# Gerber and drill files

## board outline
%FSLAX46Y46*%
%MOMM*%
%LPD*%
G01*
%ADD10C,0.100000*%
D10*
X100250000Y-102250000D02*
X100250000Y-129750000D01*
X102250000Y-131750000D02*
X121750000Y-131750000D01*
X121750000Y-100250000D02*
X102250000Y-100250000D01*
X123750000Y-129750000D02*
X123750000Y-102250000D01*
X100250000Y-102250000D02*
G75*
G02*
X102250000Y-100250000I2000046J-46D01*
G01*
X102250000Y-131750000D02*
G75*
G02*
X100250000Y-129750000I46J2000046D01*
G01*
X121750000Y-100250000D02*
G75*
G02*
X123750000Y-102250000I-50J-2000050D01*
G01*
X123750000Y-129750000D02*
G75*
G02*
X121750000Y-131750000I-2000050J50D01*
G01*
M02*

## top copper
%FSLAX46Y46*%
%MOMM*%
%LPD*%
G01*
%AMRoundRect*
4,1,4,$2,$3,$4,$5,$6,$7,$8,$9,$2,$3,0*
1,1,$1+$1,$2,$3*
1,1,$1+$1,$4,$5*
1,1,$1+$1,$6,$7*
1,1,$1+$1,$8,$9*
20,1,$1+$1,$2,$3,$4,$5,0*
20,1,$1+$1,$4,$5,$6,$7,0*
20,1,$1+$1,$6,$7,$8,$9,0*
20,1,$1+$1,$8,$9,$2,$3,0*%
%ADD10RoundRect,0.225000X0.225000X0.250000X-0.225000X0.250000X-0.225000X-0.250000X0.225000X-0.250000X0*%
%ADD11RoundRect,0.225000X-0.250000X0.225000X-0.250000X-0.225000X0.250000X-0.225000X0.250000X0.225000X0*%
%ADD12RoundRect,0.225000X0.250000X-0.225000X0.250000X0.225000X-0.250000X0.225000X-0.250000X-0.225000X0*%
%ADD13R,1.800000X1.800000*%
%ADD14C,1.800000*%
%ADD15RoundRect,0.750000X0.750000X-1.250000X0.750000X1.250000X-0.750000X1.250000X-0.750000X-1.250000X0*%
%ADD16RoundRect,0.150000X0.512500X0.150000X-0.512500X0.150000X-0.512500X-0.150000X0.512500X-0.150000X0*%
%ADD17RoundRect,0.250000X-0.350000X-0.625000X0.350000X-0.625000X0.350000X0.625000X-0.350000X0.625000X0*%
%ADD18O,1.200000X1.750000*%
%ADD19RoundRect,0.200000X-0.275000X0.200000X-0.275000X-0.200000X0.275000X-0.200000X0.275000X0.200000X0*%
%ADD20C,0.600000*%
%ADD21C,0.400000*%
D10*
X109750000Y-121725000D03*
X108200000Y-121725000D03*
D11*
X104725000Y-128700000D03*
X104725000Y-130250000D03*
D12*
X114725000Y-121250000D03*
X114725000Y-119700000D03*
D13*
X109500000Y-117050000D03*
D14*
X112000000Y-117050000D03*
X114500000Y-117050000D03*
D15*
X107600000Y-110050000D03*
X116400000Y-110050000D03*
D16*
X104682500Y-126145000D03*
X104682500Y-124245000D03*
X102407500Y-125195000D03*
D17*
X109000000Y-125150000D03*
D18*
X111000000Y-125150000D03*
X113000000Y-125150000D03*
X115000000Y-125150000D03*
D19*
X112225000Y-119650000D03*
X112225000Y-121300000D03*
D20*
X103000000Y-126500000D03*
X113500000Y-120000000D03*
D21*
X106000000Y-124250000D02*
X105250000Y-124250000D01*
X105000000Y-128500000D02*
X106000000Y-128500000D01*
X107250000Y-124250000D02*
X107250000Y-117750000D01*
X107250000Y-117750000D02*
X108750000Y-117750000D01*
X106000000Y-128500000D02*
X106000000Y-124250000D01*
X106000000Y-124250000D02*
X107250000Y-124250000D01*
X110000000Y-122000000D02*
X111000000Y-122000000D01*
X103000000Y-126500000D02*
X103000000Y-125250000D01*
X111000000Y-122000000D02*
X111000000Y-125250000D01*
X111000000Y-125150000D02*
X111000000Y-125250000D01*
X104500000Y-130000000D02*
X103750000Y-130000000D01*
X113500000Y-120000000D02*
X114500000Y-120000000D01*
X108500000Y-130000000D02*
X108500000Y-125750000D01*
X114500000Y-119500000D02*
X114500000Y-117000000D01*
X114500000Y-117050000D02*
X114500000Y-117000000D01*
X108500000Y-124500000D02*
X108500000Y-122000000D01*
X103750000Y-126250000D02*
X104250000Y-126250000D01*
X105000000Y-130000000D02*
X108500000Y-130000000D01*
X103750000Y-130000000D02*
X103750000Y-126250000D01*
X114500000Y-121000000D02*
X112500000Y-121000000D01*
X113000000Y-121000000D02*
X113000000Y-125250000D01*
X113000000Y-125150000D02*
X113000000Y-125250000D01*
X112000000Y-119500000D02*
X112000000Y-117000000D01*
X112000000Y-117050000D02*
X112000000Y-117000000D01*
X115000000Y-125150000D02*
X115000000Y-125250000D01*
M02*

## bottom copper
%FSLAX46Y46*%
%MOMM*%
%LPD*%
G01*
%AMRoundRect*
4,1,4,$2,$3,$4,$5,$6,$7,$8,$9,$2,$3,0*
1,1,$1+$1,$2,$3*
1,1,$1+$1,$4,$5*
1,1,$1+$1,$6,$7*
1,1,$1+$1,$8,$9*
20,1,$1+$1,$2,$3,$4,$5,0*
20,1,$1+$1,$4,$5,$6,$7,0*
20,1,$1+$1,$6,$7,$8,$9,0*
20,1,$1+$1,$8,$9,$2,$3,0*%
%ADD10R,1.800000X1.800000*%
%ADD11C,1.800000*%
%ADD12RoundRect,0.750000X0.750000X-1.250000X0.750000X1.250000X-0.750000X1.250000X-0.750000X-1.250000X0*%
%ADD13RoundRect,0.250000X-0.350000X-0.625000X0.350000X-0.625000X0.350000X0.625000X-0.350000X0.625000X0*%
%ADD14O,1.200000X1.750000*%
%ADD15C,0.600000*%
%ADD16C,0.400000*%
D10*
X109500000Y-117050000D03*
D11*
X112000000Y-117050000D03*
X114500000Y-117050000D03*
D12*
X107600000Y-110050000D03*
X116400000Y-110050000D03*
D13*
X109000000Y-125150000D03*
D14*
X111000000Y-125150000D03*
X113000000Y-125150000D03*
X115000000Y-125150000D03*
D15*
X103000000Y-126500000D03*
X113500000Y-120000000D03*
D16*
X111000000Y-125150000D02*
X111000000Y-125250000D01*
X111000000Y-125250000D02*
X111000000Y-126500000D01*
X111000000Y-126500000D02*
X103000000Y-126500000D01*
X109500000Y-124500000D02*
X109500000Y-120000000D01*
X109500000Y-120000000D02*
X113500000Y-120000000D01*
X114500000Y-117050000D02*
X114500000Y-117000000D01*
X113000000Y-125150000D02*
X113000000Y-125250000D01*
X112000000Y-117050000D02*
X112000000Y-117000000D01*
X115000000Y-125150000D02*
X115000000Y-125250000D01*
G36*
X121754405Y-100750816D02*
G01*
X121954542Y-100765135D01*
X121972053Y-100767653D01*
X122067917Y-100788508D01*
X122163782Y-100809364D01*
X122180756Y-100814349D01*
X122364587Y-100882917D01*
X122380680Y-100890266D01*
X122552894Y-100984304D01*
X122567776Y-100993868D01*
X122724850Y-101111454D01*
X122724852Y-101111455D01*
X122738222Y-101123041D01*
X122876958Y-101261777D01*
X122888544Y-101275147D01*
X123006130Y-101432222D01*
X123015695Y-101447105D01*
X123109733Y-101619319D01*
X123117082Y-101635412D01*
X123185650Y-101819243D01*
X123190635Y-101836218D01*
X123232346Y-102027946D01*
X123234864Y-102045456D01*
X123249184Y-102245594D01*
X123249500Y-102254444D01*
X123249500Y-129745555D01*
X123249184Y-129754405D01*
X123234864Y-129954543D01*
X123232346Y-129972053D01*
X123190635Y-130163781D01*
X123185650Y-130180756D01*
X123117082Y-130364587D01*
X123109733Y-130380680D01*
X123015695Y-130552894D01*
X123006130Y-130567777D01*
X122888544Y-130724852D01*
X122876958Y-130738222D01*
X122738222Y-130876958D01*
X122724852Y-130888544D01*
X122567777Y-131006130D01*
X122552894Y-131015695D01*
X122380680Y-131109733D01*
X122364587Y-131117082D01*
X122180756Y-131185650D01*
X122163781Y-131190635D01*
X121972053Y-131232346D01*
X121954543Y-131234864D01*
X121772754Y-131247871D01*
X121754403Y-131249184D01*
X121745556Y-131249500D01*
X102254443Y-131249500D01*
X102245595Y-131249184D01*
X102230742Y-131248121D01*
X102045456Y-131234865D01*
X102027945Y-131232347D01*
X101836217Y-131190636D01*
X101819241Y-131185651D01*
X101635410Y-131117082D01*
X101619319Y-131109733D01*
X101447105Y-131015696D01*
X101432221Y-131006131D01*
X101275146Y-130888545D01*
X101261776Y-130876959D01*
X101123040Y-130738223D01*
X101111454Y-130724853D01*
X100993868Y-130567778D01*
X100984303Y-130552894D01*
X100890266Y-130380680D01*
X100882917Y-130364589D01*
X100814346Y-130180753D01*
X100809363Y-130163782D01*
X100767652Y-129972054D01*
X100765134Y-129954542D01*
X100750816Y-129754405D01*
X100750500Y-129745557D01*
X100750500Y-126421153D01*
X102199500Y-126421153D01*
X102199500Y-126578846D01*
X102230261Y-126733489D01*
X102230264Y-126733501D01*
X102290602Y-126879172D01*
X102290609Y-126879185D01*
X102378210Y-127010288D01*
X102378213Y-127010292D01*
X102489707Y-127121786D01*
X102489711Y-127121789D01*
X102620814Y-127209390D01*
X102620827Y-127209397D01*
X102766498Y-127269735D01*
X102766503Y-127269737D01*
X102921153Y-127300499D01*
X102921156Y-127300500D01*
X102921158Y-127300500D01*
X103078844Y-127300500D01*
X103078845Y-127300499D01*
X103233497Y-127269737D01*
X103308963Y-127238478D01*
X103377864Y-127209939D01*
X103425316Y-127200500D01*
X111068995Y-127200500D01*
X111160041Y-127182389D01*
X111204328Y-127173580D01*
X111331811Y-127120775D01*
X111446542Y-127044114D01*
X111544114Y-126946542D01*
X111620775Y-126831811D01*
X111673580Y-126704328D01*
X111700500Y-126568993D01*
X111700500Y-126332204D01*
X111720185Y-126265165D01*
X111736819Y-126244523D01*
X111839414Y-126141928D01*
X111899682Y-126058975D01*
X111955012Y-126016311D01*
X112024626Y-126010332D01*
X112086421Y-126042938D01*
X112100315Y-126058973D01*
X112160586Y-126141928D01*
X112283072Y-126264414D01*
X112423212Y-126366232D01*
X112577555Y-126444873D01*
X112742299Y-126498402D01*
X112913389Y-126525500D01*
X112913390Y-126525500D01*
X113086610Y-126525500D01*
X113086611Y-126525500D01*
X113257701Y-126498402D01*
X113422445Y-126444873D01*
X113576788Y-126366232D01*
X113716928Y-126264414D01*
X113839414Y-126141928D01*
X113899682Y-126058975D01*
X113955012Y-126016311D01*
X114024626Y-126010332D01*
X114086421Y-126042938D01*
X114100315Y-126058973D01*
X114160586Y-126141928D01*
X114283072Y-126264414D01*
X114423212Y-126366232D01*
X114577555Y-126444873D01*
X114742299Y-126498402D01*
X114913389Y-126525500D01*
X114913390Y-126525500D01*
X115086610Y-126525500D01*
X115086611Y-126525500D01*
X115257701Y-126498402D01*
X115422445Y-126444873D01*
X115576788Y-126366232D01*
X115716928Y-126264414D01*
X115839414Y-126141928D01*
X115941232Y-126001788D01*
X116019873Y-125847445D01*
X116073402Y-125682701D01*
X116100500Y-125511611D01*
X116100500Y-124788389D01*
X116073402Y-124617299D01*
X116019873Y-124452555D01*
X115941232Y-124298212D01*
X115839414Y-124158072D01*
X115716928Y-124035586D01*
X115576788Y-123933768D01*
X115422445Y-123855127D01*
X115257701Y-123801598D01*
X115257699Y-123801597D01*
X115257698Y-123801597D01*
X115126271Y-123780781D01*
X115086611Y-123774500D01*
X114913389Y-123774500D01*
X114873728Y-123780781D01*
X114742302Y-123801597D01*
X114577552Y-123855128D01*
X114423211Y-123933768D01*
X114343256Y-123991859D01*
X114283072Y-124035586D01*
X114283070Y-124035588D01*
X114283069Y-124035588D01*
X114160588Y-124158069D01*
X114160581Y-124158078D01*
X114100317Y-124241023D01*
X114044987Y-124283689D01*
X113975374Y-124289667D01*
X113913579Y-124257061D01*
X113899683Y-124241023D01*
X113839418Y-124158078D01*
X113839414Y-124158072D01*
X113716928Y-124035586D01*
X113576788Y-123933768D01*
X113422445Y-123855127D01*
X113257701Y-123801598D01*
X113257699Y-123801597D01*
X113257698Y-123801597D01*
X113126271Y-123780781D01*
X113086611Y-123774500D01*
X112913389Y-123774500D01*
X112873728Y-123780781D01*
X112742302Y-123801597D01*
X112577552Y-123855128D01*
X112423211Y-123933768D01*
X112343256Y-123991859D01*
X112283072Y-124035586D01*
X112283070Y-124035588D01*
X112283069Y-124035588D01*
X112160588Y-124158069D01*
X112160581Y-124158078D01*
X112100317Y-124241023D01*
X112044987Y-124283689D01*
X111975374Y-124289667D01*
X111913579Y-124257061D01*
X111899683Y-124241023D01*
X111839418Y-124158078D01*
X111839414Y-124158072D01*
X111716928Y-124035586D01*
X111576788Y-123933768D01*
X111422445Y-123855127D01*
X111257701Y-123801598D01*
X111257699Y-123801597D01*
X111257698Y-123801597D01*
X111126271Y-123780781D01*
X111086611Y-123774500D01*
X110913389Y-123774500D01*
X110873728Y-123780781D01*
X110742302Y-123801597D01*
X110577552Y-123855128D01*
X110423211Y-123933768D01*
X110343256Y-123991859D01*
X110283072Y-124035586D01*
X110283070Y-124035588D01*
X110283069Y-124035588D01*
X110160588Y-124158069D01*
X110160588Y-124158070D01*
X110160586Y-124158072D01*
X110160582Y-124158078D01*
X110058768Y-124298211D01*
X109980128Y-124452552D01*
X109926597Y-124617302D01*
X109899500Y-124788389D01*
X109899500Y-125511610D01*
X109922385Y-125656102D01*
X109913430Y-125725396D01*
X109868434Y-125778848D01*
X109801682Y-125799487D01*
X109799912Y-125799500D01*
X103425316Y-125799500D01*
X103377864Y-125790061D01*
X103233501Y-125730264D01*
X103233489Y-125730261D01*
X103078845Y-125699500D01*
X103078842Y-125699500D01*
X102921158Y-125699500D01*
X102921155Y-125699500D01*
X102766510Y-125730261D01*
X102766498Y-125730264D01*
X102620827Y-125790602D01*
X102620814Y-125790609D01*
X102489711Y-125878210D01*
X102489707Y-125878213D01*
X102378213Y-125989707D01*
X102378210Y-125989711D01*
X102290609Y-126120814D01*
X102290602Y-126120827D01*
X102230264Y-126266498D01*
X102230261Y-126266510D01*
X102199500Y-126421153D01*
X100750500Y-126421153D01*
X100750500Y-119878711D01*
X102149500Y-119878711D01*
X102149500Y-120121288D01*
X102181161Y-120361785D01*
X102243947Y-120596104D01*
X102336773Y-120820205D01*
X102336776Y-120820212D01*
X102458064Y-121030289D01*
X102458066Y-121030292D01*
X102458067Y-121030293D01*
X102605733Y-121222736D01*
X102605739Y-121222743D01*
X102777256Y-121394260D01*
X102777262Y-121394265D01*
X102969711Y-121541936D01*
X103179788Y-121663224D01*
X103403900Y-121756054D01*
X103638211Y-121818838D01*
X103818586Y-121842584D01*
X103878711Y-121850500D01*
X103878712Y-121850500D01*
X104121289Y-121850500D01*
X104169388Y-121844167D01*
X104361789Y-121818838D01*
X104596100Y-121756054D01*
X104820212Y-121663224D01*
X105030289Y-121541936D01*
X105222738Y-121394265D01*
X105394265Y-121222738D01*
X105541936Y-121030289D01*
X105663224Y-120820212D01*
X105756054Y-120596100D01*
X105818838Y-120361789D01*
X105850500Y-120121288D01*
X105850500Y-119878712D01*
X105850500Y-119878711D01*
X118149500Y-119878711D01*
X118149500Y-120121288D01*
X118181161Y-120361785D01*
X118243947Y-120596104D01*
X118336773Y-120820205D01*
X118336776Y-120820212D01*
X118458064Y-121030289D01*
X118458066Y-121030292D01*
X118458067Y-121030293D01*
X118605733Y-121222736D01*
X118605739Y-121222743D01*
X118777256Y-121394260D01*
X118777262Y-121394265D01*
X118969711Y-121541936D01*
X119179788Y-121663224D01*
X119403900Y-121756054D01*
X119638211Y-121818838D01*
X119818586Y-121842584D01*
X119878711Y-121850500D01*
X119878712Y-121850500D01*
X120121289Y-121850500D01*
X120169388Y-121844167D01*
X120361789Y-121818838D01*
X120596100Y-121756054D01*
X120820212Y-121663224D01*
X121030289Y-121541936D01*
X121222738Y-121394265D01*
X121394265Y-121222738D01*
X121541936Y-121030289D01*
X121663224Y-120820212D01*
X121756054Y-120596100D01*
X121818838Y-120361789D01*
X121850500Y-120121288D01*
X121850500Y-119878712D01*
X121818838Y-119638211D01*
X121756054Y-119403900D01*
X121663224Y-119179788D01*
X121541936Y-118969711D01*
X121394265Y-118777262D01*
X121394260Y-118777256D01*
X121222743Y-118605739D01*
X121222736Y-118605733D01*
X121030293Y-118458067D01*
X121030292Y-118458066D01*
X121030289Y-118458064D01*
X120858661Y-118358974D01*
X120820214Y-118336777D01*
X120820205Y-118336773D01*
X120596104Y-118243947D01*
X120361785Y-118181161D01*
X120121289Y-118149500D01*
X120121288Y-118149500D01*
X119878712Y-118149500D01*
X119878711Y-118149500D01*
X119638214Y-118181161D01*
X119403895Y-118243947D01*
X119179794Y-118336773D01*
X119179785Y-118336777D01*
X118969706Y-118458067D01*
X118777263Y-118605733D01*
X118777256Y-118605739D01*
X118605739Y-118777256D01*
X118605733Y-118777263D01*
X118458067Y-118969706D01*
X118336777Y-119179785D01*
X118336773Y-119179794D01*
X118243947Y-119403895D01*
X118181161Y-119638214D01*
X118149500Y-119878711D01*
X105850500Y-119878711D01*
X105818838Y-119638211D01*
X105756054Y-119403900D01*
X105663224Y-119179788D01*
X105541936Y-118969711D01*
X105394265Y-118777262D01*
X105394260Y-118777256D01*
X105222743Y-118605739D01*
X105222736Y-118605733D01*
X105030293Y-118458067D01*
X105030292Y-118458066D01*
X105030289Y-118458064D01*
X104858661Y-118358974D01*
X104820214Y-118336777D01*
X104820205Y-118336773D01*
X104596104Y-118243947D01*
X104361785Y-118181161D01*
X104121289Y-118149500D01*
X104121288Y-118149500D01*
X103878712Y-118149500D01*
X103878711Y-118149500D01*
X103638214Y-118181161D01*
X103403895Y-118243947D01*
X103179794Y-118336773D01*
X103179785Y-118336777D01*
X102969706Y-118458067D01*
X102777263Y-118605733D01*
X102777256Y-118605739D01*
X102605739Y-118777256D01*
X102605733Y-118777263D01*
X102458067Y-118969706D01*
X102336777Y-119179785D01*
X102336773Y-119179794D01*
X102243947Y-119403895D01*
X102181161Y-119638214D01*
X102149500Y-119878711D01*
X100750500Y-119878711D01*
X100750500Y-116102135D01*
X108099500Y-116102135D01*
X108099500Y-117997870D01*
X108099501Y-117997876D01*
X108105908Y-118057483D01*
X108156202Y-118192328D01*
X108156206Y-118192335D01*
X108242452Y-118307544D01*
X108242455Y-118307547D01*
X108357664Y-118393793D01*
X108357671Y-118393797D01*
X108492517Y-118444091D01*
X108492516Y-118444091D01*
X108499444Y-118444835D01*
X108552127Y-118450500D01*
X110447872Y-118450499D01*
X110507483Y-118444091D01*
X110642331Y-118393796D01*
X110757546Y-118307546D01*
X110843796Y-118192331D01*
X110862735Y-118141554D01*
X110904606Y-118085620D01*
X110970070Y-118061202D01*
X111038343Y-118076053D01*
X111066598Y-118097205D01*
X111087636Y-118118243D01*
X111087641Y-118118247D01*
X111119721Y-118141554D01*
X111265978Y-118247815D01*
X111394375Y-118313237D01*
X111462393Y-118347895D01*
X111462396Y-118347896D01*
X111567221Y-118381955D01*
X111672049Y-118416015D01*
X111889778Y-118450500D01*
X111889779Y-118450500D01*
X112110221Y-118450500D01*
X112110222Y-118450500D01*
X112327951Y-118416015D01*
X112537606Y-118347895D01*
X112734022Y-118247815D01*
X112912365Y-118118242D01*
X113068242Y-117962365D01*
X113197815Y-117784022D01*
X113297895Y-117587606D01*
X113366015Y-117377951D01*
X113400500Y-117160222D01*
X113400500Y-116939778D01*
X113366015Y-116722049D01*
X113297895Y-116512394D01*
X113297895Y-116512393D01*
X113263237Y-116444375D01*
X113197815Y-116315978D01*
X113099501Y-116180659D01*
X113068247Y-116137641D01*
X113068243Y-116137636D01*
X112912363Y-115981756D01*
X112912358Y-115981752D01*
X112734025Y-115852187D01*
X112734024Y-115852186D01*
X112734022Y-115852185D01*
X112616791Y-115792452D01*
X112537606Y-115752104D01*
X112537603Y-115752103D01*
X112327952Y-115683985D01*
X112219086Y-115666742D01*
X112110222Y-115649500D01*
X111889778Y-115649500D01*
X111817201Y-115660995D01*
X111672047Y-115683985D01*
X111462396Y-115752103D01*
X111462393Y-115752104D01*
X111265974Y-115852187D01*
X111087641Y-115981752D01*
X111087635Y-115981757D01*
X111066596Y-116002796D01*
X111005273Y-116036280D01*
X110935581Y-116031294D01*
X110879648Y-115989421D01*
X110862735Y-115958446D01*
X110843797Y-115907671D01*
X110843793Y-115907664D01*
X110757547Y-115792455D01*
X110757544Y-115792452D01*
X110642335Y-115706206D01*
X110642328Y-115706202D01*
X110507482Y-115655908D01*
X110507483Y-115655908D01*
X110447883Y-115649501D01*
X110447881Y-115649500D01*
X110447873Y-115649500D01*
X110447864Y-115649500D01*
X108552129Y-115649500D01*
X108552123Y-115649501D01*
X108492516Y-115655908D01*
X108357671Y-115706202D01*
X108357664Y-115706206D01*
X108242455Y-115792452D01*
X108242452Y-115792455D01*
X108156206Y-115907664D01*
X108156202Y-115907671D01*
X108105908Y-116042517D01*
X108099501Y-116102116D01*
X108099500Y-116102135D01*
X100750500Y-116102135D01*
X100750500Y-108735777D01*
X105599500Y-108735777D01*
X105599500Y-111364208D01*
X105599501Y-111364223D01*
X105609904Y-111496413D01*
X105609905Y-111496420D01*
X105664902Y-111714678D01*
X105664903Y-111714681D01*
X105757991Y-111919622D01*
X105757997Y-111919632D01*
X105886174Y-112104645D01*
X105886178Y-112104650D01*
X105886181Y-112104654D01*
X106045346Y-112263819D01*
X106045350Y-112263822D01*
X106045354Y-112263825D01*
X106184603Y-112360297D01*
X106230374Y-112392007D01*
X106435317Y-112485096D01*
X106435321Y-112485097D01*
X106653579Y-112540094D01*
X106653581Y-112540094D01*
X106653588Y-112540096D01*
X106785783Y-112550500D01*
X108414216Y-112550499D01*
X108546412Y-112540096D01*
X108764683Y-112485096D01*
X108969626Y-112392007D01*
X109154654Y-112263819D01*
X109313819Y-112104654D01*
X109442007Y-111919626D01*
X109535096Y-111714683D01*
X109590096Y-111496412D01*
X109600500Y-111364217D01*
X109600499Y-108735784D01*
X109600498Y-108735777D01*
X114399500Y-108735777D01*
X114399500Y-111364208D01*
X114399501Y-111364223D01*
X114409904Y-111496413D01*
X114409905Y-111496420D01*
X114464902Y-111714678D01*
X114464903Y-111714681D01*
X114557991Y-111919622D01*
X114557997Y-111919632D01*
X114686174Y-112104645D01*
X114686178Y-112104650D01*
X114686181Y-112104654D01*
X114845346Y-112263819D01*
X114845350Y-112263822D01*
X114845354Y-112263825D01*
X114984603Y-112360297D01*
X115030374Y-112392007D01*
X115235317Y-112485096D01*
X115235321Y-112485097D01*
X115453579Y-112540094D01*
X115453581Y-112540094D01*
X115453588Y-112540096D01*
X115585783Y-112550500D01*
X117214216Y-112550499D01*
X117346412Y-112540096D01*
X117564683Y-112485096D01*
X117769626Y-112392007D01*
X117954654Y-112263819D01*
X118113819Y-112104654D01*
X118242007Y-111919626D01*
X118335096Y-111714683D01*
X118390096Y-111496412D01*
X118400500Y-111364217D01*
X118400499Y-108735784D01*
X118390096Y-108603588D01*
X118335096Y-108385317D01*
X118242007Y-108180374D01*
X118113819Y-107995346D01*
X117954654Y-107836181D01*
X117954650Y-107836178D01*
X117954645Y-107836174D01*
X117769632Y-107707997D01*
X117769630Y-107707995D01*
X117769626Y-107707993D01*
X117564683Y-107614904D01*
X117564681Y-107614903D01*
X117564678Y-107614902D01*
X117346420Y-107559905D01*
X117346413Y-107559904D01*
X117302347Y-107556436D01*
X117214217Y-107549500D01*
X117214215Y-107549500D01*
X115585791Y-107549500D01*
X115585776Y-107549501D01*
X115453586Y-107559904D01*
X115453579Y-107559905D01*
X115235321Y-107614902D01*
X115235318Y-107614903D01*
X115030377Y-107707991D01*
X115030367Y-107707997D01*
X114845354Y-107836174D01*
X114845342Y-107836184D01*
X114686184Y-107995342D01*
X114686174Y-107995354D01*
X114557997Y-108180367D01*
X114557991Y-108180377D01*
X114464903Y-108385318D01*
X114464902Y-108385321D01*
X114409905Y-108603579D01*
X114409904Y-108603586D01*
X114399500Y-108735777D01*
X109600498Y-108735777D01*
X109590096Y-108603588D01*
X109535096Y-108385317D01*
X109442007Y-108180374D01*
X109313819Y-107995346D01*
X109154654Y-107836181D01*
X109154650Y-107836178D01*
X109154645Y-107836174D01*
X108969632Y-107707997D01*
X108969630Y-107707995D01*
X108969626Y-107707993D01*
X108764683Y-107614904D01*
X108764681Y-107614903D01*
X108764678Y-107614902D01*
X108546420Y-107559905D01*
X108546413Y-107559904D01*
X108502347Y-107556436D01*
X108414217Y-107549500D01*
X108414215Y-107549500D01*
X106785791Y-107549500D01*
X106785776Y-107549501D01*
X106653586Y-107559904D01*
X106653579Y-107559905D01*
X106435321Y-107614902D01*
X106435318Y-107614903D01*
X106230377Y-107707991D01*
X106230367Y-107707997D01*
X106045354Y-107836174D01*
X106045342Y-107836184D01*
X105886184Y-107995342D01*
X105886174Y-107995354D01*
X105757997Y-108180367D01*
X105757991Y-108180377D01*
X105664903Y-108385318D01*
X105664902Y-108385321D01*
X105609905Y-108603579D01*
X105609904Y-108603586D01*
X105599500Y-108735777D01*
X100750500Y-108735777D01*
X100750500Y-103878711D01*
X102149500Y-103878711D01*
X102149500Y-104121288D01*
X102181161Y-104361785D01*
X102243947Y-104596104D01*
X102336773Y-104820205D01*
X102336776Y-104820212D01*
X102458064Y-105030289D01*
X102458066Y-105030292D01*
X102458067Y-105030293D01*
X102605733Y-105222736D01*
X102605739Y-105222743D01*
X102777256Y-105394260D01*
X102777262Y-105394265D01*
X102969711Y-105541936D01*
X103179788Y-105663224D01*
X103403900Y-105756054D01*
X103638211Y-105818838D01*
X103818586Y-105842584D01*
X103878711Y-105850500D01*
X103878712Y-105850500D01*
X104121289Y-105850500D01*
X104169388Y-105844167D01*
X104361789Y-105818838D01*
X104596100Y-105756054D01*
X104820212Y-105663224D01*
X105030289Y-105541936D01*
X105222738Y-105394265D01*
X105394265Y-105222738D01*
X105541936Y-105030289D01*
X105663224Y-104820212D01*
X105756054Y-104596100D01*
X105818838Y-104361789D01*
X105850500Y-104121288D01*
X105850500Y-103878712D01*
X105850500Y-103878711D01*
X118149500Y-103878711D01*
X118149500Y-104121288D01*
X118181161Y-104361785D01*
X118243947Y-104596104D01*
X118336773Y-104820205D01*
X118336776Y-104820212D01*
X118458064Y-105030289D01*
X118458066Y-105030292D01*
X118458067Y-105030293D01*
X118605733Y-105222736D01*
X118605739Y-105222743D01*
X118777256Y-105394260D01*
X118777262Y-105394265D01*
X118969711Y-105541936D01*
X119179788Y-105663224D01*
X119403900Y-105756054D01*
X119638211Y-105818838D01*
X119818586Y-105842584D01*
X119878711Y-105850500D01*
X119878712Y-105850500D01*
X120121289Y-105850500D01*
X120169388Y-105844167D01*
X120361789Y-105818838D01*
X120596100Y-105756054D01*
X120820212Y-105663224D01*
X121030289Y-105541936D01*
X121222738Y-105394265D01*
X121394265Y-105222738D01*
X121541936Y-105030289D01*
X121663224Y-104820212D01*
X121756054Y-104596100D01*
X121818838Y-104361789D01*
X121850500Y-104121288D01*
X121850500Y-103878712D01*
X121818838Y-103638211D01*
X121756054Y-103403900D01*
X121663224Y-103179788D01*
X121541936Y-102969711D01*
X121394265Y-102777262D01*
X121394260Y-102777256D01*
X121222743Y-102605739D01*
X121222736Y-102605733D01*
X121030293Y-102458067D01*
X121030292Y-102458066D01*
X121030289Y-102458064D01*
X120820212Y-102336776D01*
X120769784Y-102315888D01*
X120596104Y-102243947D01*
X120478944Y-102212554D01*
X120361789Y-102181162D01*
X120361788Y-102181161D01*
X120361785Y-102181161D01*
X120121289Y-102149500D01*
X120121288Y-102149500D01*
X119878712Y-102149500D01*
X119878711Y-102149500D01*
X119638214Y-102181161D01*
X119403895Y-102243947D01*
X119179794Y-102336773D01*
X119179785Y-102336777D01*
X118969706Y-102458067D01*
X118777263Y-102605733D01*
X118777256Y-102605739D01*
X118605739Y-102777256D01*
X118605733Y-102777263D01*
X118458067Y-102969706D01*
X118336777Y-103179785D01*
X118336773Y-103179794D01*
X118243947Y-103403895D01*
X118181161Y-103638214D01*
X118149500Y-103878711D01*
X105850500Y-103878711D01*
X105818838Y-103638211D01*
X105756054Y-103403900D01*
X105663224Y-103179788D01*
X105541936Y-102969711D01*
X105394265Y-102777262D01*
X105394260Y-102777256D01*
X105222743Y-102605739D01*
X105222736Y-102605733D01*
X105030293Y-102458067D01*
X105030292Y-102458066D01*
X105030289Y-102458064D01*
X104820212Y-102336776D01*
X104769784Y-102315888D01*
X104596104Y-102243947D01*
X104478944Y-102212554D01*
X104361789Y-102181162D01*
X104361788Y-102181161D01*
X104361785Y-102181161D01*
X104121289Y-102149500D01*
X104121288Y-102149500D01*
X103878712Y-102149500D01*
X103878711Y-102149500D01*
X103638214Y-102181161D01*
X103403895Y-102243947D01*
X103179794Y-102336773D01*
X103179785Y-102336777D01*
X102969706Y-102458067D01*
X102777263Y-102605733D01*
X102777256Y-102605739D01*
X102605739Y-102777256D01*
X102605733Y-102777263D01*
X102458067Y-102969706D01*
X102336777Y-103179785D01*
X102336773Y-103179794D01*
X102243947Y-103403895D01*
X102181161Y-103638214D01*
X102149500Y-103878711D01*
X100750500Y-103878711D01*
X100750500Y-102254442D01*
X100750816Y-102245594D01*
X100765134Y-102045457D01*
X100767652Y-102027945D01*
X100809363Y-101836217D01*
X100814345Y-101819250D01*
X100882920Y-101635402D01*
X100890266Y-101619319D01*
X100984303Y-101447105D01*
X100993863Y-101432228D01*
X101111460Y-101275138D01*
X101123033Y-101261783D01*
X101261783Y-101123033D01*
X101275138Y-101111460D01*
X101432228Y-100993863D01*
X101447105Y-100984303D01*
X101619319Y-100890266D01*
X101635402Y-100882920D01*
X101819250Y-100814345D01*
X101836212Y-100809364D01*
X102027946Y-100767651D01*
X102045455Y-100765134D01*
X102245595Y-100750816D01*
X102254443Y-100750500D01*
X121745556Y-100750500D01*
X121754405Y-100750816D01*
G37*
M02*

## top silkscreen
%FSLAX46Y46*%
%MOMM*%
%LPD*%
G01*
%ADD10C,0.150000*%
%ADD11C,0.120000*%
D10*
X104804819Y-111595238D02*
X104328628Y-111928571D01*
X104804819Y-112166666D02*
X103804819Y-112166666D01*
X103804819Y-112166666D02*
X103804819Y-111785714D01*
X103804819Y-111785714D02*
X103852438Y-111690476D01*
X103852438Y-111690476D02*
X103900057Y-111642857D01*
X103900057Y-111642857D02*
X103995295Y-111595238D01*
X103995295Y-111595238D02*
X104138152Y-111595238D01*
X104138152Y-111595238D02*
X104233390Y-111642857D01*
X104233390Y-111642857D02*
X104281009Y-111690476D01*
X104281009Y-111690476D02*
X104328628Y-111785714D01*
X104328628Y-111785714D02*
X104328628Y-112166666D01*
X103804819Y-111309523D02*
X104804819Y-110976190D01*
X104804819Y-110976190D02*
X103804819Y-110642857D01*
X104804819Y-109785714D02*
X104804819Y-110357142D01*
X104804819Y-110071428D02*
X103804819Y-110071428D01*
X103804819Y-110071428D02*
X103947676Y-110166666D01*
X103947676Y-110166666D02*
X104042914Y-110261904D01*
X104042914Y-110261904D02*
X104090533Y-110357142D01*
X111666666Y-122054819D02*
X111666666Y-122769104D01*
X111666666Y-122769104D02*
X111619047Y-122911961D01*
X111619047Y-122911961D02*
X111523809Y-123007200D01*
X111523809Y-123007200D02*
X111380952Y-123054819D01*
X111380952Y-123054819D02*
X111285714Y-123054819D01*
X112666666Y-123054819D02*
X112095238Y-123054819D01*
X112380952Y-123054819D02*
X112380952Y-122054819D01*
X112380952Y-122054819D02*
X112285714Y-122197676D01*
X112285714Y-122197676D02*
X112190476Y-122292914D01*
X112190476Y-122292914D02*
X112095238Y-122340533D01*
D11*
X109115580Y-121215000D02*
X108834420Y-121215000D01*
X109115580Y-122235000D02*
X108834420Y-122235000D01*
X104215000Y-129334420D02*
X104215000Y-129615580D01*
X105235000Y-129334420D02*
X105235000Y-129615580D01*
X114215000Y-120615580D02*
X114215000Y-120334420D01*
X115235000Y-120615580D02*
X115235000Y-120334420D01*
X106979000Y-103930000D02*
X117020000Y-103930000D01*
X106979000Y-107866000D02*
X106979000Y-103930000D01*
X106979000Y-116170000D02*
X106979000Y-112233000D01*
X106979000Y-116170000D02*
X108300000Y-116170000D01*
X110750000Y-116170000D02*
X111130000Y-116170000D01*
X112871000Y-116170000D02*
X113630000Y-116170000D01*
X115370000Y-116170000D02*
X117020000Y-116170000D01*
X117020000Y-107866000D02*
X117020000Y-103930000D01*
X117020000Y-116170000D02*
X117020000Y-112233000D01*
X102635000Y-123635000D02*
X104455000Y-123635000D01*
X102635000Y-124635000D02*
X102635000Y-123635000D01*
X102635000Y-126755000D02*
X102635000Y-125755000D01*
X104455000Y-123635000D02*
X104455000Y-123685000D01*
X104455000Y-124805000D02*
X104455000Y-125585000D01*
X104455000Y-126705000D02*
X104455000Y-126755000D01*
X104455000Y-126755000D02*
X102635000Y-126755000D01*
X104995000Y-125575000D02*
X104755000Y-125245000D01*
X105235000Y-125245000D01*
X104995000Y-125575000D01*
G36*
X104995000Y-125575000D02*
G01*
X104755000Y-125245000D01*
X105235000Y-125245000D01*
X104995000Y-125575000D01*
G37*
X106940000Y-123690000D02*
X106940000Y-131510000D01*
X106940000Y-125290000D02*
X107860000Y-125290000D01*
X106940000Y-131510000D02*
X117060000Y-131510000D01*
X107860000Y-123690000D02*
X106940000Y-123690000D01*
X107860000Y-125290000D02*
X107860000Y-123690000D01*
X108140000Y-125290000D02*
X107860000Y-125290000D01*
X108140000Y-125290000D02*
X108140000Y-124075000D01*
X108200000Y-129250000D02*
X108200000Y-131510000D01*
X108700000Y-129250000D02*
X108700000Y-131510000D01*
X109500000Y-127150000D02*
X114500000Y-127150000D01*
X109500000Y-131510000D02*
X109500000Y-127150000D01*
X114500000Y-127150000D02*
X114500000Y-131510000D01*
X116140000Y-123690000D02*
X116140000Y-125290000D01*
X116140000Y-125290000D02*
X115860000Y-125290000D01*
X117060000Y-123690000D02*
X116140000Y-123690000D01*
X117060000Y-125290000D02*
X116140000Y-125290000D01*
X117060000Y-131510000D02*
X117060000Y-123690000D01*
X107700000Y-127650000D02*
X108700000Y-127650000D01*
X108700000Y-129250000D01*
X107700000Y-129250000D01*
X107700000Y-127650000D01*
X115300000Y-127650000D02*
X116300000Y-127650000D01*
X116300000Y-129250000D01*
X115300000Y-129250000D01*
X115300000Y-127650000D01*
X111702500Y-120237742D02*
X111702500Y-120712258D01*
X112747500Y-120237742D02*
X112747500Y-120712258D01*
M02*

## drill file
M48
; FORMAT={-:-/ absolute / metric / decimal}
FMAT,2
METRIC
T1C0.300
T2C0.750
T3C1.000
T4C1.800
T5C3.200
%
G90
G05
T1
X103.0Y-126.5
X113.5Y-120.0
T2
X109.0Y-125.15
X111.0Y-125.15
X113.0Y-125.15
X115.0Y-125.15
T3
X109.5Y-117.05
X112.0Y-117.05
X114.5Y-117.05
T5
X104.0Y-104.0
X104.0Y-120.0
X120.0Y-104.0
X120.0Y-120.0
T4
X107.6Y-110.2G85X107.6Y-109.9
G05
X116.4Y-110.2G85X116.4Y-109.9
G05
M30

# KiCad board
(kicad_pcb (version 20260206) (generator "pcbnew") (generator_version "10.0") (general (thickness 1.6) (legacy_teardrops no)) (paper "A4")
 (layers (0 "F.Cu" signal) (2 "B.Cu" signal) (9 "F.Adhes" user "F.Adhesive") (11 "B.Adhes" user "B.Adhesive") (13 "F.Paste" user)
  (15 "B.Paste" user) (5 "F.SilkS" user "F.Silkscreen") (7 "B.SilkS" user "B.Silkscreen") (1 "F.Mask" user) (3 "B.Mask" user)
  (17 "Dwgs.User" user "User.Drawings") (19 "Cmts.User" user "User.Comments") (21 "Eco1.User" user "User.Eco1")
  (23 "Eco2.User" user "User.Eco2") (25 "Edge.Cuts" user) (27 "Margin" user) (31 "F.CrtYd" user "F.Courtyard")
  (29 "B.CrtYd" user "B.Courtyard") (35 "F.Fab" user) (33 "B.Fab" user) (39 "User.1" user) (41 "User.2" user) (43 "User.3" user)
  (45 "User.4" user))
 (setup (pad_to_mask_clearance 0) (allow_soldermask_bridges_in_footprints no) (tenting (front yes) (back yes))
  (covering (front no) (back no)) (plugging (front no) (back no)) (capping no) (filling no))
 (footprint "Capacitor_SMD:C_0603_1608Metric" (layer "F.Cu") (at 108.975 121.725 180)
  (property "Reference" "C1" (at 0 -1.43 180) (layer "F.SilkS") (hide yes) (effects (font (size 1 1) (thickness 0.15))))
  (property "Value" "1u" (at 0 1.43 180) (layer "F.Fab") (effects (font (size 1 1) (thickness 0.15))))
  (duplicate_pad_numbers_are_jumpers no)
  (fp_line (start -0.14058 0.51) (end 0.14058 0.51) (stroke (width 0.12) (type solid)) (layer "F.SilkS"))
  (fp_line (start -0.14058 -0.51) (end 0.14058 -0.51) (stroke (width 0.12) (type solid)) (layer "F.SilkS"))
  (pad "1" smd roundrect (at -0.775 0 180) (size 0.9 0.95) (layers "F.Cu" "F.Mask" "F.Paste") (roundrect_rratio 0.25) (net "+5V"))
  (pad "2" smd roundrect (at 0.775 0 180) (size 0.9 0.95) (layers "F.Cu" "F.Mask" "F.Paste") (roundrect_rratio 0.25) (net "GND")))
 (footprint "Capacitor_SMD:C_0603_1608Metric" (layer "F.Cu") (at 104.725 129.475 -90)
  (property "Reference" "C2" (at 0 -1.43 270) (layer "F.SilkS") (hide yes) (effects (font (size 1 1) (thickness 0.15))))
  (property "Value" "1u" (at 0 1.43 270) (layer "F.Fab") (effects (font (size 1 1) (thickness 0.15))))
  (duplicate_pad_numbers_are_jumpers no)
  (fp_line (start -0.14058 0.51) (end 0.14058 0.51) (stroke (width 0.12) (type solid)) (layer "F.SilkS"))
  (fp_line (start -0.14058 -0.51) (end 0.14058 -0.51) (stroke (width 0.12) (type solid)) (layer "F.SilkS"))
  (pad "1" smd roundrect (at -0.775 0 270) (size 0.9 0.95) (layers "F.Cu" "F.Mask" "F.Paste") (roundrect_rratio 0.25) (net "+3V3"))
  (pad "2" smd roundrect (at 0.775 0 270) (size 0.9 0.95) (layers "F.Cu" "F.Mask" "F.Paste") (roundrect_rratio 0.25) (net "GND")))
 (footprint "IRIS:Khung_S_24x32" (layer "F.Cu") (at 100 132)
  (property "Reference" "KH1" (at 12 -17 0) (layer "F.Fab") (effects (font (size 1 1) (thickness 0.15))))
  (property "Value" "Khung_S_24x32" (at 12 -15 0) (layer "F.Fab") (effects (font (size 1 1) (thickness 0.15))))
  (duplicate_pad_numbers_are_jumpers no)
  (fp_line (start 0.25 -29.75) (end 0.25 -2.25) (stroke (width 0.1) (type solid)) (layer "Edge.Cuts"))
  (fp_line (start 2.25 -0.25) (end 21.75 -0.25) (stroke (width 0.1) (type solid)) (layer "Edge.Cuts"))
  (fp_line (start 21.75 -31.75) (end 2.25 -31.75) (stroke (width 0.1) (type solid)) (layer "Edge.Cuts"))
  (fp_line (start 23.75 -2.25) (end 23.75 -29.75) (stroke (width 0.1) (type solid)) (layer "Edge.Cuts"))
  (fp_arc (start 0.25 -29.75) (mid 0.8358 -31.1642) (end 2.25 -31.75) (stroke (width 0.1) (type solid)) (layer "Edge.Cuts"))
  (fp_arc (start 2.25 -0.25) (mid 0.8358 -0.8358) (end 0.25 -2.25) (stroke (width 0.1) (type solid)) (layer "Edge.Cuts"))
  (fp_arc (start 21.75 -31.75) (mid 23.164199 -31.164199) (end 23.75 -29.75) (stroke (width 0.1) (type solid)) (layer "Edge.Cuts"))
  (fp_arc (start 23.75 -2.25) (mid 23.164199 -0.835801) (end 21.75 -0.25) (stroke (width 0.1) (type solid)) (layer "Edge.Cuts"))
  (pad "" np_thru_hole circle (at 4 -28) (size 3.2 3.2) (drill 3.2) (layers "*.Cu" "*.Mask"))
  (pad "" np_thru_hole circle (at 4 -12) (size 3.2 3.2) (drill 3.2) (layers "*.Cu" "*.Mask"))
  (pad "" np_thru_hole circle (at 20 -28) (size 3.2 3.2) (drill 3.2) (layers "*.Cu" "*.Mask"))
  (pad "" np_thru_hole circle (at 20 -12) (size 3.2 3.2) (drill 3.2) (layers "*.Cu" "*.Mask")))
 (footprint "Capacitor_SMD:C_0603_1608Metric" (layer "F.Cu") (at 114.725 120.475 90)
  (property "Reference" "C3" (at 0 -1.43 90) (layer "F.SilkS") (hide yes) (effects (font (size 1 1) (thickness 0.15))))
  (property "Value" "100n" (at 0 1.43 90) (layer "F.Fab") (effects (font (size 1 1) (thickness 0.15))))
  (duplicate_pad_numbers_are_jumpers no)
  (fp_line (start -0.14058 -0.51) (end 0.14058 -0.51) (stroke (width 0.12) (type solid)) (layer "F.SilkS"))
  (fp_line (start -0.14058 0.51) (end 0.14058 0.51) (stroke (width 0.12) (type solid)) (layer "F.SilkS"))
  (pad "1" smd roundrect (at -0.775 0 90) (size 0.9 0.95) (layers "F.Cu" "F.Mask" "F.Paste") (roundrect_rratio 0.25) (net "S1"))
  (pad "2" smd roundrect (at 0.775 0 90) (size 0.9 0.95) (layers "F.Cu" "F.Mask" "F.Paste") (roundrect_rratio 0.25) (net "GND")))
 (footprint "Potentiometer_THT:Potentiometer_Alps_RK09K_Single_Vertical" (layer "F.Cu") (at 109.5 117.05 90)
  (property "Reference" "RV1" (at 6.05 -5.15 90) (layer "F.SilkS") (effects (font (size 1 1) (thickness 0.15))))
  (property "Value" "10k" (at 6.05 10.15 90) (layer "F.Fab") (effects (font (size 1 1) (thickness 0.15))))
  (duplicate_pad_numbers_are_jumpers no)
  (fp_line (start 13.12 -2.521) (end 13.12 7.52) (stroke (width 0.12) (type solid)) (layer "F.SilkS"))
  (fp_line (start 9.184 -2.521) (end 13.12 -2.521) (stroke (width 0.12) (type solid)) (layer "F.SilkS"))
  (fp_line (start 0.88 -2.521) (end 4.817 -2.521) (stroke (width 0.12) (type solid)) (layer "F.SilkS"))
  (fp_line (start 0.88 -2.521) (end 0.88 -1.2) (stroke (width 0.12) (type solid)) (layer "F.SilkS"))
  (fp_line (start 0.88 1.25) (end 0.88 1.63) (stroke (width 0.12) (type solid)) (layer "F.SilkS"))
  (fp_line (start 0.88 3.371) (end 0.88 4.13) (stroke (width 0.12) (type solid)) (layer "F.SilkS"))
  (fp_line (start 0.88 5.87) (end 0.88 7.52) (stroke (width 0.12) (type solid)) (layer "F.SilkS"))
  (fp_line (start 9.184 7.52) (end 13.12 7.52) (stroke (width 0.12) (type solid)) (layer "F.SilkS"))
  (fp_line (start 0.88 7.52) (end 4.817 7.52) (stroke (width 0.12) (type solid)) (layer "F.SilkS"))
  (pad "1" thru_hole rect (at 0 0 90) (size 1.8 1.8) (drill 1) (layers "*.Cu" "*.Mask") (remove_unused_layers no) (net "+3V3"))
  (pad "2" thru_hole circle (at 0 2.5 90) (size 1.8 1.8) (drill 1) (layers "*.Cu" "*.Mask") (remove_unused_layers no) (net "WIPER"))
  (pad "3" thru_hole circle (at 0 5 90) (size 1.8 1.8) (drill 1) (layers "*.Cu" "*.Mask") (remove_unused_layers no) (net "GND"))
  (pad "MP" thru_hole roundrect (at 7 -1.9 90) (size 4 3) (drill oval 2.1 1.8) (layers "*.Cu" "*.Mask") (remove_unused_layers no)
   (roundrect_rratio 0.25))
  (pad "MP" thru_hole roundrect (at 7 6.9 90) (size 4 3) (drill oval 2.1 1.8) (layers "*.Cu" "*.Mask") (remove_unused_layers no)
   (roundrect_rratio 0.25)))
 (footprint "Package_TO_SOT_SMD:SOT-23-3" (layer "F.Cu") (at 103.545 125.195 180)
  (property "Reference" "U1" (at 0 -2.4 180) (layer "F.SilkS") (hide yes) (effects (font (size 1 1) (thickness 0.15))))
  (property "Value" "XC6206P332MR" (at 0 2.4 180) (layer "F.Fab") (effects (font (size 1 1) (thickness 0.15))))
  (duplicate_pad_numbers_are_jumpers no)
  (fp_line (start 0.91 1.56) (end -0.91 1.56) (stroke (width 0.12) (type solid)) (layer "F.SilkS"))
  (fp_line (start 0.91 0.56) (end 0.91 1.56) (stroke (width 0.12) (type solid)) (layer "F.SilkS"))
  (fp_line (start 0.91 -1.56) (end 0.91 -0.56) (stroke (width 0.12) (type solid)) (layer "F.SilkS"))
  (fp_line (start -0.91 1.56) (end -0.91 1.51) (stroke (width 0.12) (type solid)) (layer "F.SilkS"))
  (fp_line (start -0.91 0.39) (end -0.91 -0.39) (stroke (width 0.12) (type solid)) (layer "F.SilkS"))
  (fp_line (start -0.91 -1.51) (end -0.91 -1.56) (stroke (width 0.12) (type solid)) (layer "F.SilkS"))
  (fp_line (start -0.91 -1.56) (end 0.91 -1.56) (stroke (width 0.12) (type solid)) (layer "F.SilkS"))
  (fp_poly (pts (xy -1.45 -0.38) (xy -1.21 -0.05) (xy -1.69 -0.05)) (stroke (width 0.12) (type solid)) (fill yes) (layer "F.SilkS"))
  (pad "1" smd roundrect (at -1.1375 -0.95 180) (size 1.325 0.6) (layers "F.Cu" "F.Mask" "F.Paste") (roundrect_rratio 0.25) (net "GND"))
  (pad "2" smd roundrect (at -1.1375 0.95 180) (size 1.325 0.6) (layers "F.Cu" "F.Mask" "F.Paste") (roundrect_rratio 0.25) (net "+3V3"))
  (pad "3" smd roundrect (at 1.1375 0 180) (size 1.325 0.6) (layers "F.Cu" "F.Mask" "F.Paste") (roundrect_rratio 0.25) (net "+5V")))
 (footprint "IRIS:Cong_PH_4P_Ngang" (layer "F.Cu") (at 109 125.15)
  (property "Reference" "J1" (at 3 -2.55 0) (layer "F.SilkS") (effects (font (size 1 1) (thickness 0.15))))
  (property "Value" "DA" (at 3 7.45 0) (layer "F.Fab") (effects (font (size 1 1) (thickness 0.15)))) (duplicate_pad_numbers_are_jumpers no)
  (fp_line (start -2.06 -1.46) (end -2.06 6.36) (stroke (width 0.12) (type solid)) (layer "F.SilkS"))
  (fp_line (start -2.06 0.14) (end -1.14 0.14) (stroke (width 0.12) (type solid)) (layer "F.SilkS"))
  (fp_line (start -2.06 6.36) (end 8.06 6.36) (stroke (width 0.12) (type solid)) (layer "F.SilkS"))
  (fp_line (start -1.14 -1.46) (end -2.06 -1.46) (stroke (width 0.12) (type solid)) (layer "F.SilkS"))
  (fp_line (start -1.14 0.14) (end -1.14 -1.46) (stroke (width 0.12) (type solid)) (layer "F.SilkS"))
  (fp_line (start -0.86 0.14) (end -1.14 0.14) (stroke (width 0.12) (type solid)) (layer "F.SilkS"))
  (fp_line (start -0.86 0.14) (end -0.86 -1.075) (stroke (width 0.12) (type solid)) (layer "F.SilkS"))
  (fp_line (start -0.8 4.1) (end -0.8 6.36) (stroke (width 0.12) (type solid)) (layer "F.SilkS"))
  (fp_line (start -0.3 4.1) (end -0.3 6.36) (stroke (width 0.12) (type solid)) (layer "F.SilkS"))
  (fp_line (start 0.5 2) (end 5.5 2) (stroke (width 0.12) (type solid)) (layer "F.SilkS"))
  (fp_line (start 0.5 6.36) (end 0.5 2) (stroke (width 0.12) (type solid)) (layer "F.SilkS"))
  (fp_line (start 5.5 2) (end 5.5 6.36) (stroke (width 0.12) (type solid)) (layer "F.SilkS"))
  (fp_line (start 7.14 -1.46) (end 7.14 0.14) (stroke (width 0.12) (type solid)) (layer "F.SilkS"))
  (fp_line (start 7.14 0.14) (end 6.86 0.14) (stroke (width 0.12) (type solid)) (layer "F.SilkS"))
  (fp_line (start 8.06 -1.46) (end 7.14 -1.46) (stroke (width 0.12) (type solid)) (layer "F.SilkS"))
  (fp_line (start 8.06 0.14) (end 7.14 0.14) (stroke (width 0.12) (type solid)) (layer "F.SilkS"))
  (fp_line (start 8.06 6.36) (end 8.06 -1.46) (stroke (width 0.12) (type solid)) (layer "F.SilkS"))
  (fp_rect (start -1.3 2.5) (end -0.3 4.1) (stroke (width 0.12) (type solid)) (fill no) (layer "F.SilkS"))
  (fp_rect (start 6.3 2.5) (end 7.3 4.1) (stroke (width 0.12) (type solid)) (fill no) (layer "F.SilkS"))
  (pad "1" thru_hole roundrect (at 0 0) (size 1.2 1.75) (drill 0.75) (layers "*.Cu" "*.Mask") (remove_unused_layers no)
   (roundrect_rratio 0.208333) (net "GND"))
  (pad "2" thru_hole oval (at 2 0) (size 1.2 1.75) (drill 0.75) (layers "*.Cu" "*.Mask") (remove_unused_layers no) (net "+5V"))
  (pad "3" thru_hole oval (at 4 0) (size 1.2 1.75) (drill 0.75) (layers "*.Cu" "*.Mask") (remove_unused_layers no) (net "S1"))
  (pad "4" thru_hole oval (at 6 0) (size 1.2 1.75) (drill 0.75) (layers "*.Cu" "*.Mask") (remove_unused_layers no)
   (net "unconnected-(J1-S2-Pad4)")))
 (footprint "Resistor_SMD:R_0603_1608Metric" (layer "F.Cu") (at 112.225 120.475 -90)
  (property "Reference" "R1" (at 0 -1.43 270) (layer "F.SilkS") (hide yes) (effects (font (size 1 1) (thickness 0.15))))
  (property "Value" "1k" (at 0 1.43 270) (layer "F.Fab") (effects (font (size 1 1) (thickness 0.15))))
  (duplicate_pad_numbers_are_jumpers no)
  (fp_line (start -0.237258 0.5225) (end 0.237258 0.5225) (stroke (width 0.12) (type solid)) (layer "F.SilkS"))
  (fp_line (start -0.237258 -0.5225) (end 0.237258 -0.5225) (stroke (width 0.12) (type solid)) (layer "F.SilkS"))
  (pad "1" smd roundrect (at -0.825 0 270) (size 0.8 0.95) (layers "F.Cu" "F.Mask" "F.Paste") (roundrect_rratio 0.25) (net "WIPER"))
  (pad "2" smd roundrect (at 0.825 0 270) (size 0.8 0.95) (layers "F.Cu" "F.Mask" "F.Paste") (roundrect_rratio 0.25) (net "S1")))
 (segment (start 106 124.25) (end 105.25 124.25) (width 0.4) (layer "F.Cu") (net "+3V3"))
 (segment (start 105 128.5) (end 106 128.5) (width 0.4) (layer "F.Cu") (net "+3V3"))
 (segment (start 107.25 124.25) (end 107.25 117.75) (width 0.4) (layer "F.Cu") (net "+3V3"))
 (segment (start 107.25 117.75) (end 108.75 117.75) (width 0.4) (layer "F.Cu") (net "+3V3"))
 (segment (start 106 128.5) (end 106 124.25) (width 0.4) (layer "F.Cu") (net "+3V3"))
 (segment (start 106 124.25) (end 107.25 124.25) (width 0.4) (layer "F.Cu") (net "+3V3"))
 (segment (start 110 122) (end 111 122) (width 0.4) (layer "F.Cu") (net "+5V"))
 (segment (start 103 126.5) (end 103 125.25) (width 0.4) (layer "F.Cu") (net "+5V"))
 (segment (start 111 122) (end 111 125.25) (width 0.4) (layer "F.Cu") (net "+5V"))
 (segment (start 111 125.15) (end 111 125.25) (width 0.4) (layer "F.Cu") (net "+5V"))
 (via (at 103 126.5) (size 0.6) (drill 0.3) (layers "F.Cu" "B.Cu") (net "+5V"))
 (segment (start 111 125.15) (end 111 125.25) (width 0.4) (layer "B.Cu") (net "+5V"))
 (segment (start 111 125.25) (end 111 126.5) (width 0.4) (layer "B.Cu") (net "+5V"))
 (segment (start 111 126.5) (end 103 126.5) (width 0.4) (layer "B.Cu") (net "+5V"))
 (segment (start 104.5 130) (end 103.75 130) (width 0.4) (layer "F.Cu") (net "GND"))
 (segment (start 113.5 120) (end 114.5 120) (width 0.4) (layer "F.Cu") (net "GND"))
 (segment (start 108.5 130) (end 108.5 125.75) (width 0.4) (layer "F.Cu") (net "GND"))
 (segment (start 114.5 119.5) (end 114.5 117) (width 0.4) (layer "F.Cu") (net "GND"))
 (segment (start 114.5 117.05) (end 114.5 117) (width 0.4) (layer "F.Cu") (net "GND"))
 (segment (start 108.5 124.5) (end 108.5 122) (width 0.4) (layer "F.Cu") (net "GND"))
 (segment (start 103.75 126.25) (end 104.25 126.25) (width 0.4) (layer "F.Cu") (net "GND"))
 (segment (start 105 130) (end 108.5 130) (width 0.4) (layer "F.Cu") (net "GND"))
 (segment (start 103.75 130) (end 103.75 126.25) (width 0.4) (layer "F.Cu") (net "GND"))
 (via (at 113.5 120) (size 0.6) (drill 0.3) (layers "F.Cu" "B.Cu") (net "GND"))
 (segment (start 109.5 124.5) (end 109.5 120) (width 0.4) (layer "B.Cu") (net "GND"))
 (segment (start 109.5 120) (end 113.5 120) (width 0.4) (layer "B.Cu") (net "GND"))
 (segment (start 114.5 117.05) (end 114.5 117) (width 0.4) (layer "B.Cu") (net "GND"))
 (segment (start 114.5 121) (end 112.5 121) (width 0.4) (layer "F.Cu") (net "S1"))
 (segment (start 113 121) (end 113 125.25) (width 0.4) (layer "F.Cu") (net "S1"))
 (segment (start 113 125.15) (end 113 125.25) (width 0.4) (layer "F.Cu") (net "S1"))
 (segment (start 113 125.15) (end 113 125.25) (width 0.4) (layer "B.Cu") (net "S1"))
 (segment (start 112 119.5) (end 112 117) (width 0.4) (layer "F.Cu") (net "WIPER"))
 (segment (start 112 117.05) (end 112 117) (width 0.4) (layer "F.Cu") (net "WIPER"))
 (segment (start 112 117.05) (end 112 117) (width 0.4) (layer "B.Cu") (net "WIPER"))
 (segment (start 115 125.15) (end 115 125.25) (width 0.4) (layer "F.Cu") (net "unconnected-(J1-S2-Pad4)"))
 (segment (start 115 125.15) (end 115 125.25) (width 0.4) (layer "B.Cu") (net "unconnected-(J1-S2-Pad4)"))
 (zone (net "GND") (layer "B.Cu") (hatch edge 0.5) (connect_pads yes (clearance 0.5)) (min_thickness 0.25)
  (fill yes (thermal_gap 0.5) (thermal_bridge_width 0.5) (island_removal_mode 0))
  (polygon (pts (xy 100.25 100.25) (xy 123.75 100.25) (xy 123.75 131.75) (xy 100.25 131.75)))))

